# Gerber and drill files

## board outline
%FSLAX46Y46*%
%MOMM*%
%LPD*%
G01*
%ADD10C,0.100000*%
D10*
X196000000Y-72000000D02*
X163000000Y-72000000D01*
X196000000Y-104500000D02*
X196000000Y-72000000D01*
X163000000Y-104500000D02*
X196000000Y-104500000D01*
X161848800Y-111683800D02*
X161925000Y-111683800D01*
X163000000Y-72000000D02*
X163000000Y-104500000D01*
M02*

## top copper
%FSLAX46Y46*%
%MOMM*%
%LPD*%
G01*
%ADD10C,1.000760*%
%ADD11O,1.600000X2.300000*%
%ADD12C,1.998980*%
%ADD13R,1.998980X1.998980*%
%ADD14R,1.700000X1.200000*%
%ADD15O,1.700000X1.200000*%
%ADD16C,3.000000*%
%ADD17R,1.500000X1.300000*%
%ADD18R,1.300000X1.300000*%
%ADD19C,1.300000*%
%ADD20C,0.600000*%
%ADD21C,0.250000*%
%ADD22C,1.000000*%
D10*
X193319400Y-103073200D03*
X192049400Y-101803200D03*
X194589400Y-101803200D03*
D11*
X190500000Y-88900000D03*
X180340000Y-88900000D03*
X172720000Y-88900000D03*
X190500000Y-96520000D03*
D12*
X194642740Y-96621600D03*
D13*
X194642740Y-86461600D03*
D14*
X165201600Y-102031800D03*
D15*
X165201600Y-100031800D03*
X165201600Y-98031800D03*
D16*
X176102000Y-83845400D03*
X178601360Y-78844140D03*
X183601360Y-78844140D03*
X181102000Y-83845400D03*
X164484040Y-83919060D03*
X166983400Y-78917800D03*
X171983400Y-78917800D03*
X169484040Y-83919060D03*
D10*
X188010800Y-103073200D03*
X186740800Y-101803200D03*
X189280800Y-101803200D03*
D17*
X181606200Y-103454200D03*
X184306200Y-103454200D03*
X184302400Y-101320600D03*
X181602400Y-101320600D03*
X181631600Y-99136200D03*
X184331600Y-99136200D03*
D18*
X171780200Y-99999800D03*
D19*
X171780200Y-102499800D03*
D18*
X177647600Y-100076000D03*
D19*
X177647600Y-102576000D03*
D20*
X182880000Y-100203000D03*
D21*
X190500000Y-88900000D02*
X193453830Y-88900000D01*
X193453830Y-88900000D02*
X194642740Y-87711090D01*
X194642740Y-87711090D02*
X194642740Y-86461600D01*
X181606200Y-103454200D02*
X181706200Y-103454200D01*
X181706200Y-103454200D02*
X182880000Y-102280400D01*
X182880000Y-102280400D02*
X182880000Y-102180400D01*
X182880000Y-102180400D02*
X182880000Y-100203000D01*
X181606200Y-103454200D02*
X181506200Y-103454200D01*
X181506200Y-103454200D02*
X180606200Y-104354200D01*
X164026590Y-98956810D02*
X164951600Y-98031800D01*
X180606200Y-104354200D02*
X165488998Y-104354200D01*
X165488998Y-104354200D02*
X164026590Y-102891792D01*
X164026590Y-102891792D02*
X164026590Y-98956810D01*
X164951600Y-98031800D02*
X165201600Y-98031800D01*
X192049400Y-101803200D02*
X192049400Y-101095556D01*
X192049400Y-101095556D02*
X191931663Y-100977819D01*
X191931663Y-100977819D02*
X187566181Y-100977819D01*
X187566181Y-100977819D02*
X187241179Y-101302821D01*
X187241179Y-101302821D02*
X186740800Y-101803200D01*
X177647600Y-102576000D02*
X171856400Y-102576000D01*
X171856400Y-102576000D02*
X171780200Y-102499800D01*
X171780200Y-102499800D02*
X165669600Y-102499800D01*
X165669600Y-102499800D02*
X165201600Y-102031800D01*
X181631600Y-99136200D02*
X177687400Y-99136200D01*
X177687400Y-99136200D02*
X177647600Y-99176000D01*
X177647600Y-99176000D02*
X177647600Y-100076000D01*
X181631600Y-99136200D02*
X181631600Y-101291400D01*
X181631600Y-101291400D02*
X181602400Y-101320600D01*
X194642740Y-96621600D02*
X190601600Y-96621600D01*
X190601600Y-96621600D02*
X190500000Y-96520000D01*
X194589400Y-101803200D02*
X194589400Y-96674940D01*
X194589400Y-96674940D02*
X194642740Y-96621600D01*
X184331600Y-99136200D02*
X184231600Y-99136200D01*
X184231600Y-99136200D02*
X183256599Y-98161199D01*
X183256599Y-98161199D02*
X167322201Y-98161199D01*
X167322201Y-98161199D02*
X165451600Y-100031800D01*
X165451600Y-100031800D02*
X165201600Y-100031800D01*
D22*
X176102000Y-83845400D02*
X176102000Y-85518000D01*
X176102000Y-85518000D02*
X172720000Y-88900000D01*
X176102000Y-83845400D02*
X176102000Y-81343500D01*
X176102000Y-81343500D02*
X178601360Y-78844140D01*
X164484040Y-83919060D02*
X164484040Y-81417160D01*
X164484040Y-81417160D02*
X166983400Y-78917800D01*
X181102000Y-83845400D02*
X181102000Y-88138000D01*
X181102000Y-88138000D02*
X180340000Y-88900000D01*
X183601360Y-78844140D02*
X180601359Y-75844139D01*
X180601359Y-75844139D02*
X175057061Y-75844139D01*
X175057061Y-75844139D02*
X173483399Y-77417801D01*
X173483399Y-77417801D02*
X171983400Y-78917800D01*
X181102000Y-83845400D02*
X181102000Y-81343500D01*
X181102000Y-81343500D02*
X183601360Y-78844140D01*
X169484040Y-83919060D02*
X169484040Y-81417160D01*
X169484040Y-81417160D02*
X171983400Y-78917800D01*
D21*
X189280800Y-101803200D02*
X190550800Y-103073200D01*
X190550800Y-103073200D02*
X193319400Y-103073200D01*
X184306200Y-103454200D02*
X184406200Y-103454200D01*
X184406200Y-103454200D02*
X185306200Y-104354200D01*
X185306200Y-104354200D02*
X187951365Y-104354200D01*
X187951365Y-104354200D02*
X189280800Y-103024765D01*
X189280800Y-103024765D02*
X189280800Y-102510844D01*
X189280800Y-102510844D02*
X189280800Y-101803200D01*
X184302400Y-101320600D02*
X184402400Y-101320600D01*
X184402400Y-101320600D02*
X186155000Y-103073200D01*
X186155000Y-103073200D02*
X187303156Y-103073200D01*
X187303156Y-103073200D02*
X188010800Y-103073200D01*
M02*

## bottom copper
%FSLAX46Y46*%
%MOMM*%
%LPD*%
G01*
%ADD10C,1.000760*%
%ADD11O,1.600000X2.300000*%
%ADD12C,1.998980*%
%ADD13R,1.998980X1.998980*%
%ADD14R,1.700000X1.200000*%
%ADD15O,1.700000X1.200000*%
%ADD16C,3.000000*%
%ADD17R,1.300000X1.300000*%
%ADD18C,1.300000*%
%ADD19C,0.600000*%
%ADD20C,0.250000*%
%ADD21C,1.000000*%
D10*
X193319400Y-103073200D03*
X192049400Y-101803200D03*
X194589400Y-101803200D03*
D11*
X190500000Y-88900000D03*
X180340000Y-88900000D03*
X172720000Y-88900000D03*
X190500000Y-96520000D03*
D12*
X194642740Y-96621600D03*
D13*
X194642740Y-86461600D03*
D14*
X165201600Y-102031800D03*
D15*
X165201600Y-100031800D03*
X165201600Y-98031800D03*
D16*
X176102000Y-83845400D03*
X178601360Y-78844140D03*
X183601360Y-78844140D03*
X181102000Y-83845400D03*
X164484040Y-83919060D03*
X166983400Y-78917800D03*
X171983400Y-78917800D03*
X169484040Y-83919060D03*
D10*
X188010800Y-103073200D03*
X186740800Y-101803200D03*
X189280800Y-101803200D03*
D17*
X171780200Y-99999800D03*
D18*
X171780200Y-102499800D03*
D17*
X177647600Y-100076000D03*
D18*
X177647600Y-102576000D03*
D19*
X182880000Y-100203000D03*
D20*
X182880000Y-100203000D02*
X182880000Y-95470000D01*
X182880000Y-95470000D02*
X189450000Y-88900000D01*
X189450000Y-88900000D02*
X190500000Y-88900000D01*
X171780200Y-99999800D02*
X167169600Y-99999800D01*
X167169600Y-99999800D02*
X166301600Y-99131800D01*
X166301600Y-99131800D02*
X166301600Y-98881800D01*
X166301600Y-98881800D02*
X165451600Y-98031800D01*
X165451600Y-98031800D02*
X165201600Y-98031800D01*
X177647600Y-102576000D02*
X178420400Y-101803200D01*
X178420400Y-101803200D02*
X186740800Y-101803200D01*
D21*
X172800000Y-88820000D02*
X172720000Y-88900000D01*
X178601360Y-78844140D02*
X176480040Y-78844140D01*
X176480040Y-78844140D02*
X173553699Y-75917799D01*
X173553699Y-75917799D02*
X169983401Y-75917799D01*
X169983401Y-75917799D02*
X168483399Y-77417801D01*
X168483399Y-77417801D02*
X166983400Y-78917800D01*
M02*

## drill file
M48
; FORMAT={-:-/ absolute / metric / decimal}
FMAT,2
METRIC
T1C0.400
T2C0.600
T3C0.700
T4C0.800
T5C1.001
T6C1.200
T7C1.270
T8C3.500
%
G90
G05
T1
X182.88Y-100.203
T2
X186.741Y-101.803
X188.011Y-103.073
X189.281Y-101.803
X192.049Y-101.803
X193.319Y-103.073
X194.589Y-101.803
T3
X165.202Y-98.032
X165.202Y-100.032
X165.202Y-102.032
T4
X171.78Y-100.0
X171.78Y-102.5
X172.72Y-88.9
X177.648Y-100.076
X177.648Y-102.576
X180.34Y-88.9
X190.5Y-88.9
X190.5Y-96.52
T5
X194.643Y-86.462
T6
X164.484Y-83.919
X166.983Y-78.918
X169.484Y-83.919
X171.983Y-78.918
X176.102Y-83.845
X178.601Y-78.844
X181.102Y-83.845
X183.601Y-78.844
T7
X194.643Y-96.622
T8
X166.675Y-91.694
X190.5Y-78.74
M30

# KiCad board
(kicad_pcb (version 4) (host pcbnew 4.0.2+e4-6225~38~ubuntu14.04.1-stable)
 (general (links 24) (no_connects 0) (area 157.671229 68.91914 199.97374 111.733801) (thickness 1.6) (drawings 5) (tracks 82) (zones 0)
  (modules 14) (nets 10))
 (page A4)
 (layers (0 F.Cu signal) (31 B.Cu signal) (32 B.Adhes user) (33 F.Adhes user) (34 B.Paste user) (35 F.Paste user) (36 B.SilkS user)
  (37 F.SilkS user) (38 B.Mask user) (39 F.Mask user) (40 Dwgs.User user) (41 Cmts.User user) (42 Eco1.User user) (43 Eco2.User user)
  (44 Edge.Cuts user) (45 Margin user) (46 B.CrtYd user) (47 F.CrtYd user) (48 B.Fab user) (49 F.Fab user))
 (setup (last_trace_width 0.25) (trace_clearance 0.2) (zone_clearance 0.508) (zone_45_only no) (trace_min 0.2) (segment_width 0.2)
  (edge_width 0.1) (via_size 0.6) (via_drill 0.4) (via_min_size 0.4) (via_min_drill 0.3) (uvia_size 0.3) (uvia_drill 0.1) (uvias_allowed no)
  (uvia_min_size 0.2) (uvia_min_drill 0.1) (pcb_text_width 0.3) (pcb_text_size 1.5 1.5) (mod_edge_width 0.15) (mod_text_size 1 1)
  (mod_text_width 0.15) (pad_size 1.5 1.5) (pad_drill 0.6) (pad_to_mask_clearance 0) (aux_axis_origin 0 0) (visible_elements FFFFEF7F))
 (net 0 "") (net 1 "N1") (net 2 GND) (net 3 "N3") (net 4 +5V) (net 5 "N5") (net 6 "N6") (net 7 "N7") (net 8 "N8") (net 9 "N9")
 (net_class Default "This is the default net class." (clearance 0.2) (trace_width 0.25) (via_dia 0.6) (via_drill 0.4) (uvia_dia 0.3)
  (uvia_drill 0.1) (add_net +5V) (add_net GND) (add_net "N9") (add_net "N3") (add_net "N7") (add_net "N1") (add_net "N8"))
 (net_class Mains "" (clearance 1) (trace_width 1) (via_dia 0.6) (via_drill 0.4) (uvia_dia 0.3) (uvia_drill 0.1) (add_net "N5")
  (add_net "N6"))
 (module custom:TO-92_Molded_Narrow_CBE (layer F.Cu) (at 194.5894 101.8032 180)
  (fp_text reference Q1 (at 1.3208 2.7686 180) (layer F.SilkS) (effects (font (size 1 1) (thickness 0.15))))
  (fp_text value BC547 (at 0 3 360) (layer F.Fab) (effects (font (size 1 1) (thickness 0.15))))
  (pad 2 thru_hole circle (at 1.27 -1.27 270) (size 1.00076 1.00076) (drill 0.6) (layers *.Cu *.Mask F.SilkS) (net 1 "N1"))
  (pad 3 thru_hole circle (at 2.54 0 270) (size 1.00076 1.00076) (drill 0.6) (layers *.Cu *.Mask F.SilkS) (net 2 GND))
  (pad 1 thru_hole circle (at 0 0 270) (size 1.00076 1.00076) (drill 0.6) (layers *.Cu *.Mask F.SilkS) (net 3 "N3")))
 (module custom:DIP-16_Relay (layer F.Cu) (at 190.5 88.9 270)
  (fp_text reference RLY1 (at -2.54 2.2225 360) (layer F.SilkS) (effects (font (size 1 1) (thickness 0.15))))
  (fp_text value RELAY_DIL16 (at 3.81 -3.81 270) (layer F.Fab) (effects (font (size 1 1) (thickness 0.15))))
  (pad 1 thru_hole oval (at 0 0 270) (size 2.3 1.6) (drill 0.8) (layers *.Cu *.Mask F.SilkS) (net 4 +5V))
  (pad 5 thru_hole oval (at 0 10.16 270) (size 2.3 1.6) (drill 0.8) (layers *.Cu *.Mask F.SilkS) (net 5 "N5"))
  (pad 8 thru_hole oval (at 0 17.78 270) (size 2.3 1.6) (drill 0.8) (layers *.Cu *.Mask F.SilkS) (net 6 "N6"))
  (pad 16 thru_hole oval (at 7.62 0 270) (size 2.3 1.6) (drill 0.8) (layers *.Cu *.Mask F.SilkS) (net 3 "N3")))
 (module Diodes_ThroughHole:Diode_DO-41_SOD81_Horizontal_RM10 (layer F.Cu) (at 194.6402 86.4616 270)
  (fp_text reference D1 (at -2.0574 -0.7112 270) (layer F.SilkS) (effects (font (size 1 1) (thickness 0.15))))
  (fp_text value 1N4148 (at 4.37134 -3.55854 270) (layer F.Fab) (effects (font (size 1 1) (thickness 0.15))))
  (pad 2 thru_hole circle (at 10.16 -0.00254 90) (size 1.99898 1.99898) (drill 1.27) (layers *.Cu *.Mask F.SilkS) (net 3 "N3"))
  (pad 1 thru_hole rect (at 0 -0.00254 90) (size 1.99898 1.99898) (drill 1.00076) (layers *.Cu *.Mask F.SilkS) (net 4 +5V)))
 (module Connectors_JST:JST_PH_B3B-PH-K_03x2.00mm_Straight (layer F.Cu) (at 165.2016 102.0318 90)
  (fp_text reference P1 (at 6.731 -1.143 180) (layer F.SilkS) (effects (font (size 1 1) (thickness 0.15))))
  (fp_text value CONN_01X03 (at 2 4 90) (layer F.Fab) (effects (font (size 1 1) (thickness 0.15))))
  (pad 1 thru_hole rect (at 0 0 90) (size 1.2 1.7) (drill 0.7) (layers *.Cu *.Mask F.SilkS) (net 2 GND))
  (pad 2 thru_hole oval (at 2 0 90) (size 1.2 1.7) (drill 0.7) (layers *.Cu *.Mask F.SilkS) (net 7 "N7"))
  (pad 3 thru_hole oval (at 4 0 90) (size 1.2 1.7) (drill 0.7) (layers *.Cu *.Mask F.SilkS) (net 4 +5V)))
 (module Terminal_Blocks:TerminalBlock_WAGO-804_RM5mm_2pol (layer F.Cu) (at 183.60136 78.84414 180)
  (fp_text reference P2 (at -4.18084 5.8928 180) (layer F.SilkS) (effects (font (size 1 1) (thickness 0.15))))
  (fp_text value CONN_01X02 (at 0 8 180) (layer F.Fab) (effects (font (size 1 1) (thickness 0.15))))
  (pad 2 thru_hole circle (at 7.49936 -5.00126 180) (size 3 3) (drill 1.2) (layers *.Cu *.Mask F.SilkS) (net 6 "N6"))
  (pad 2 thru_hole circle (at 5 0 180) (size 3 3) (drill 1.2) (layers *.Cu *.Mask F.SilkS) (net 6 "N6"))
  (pad 1 thru_hole circle (at 0 0 180) (size 3 3) (drill 1.2) (layers *.Cu *.Mask F.SilkS) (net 5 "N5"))
  (pad 1 thru_hole circle (at 2.49936 -5.00126 180) (size 3 3) (drill 1.2) (layers *.Cu *.Mask F.SilkS) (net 5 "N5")))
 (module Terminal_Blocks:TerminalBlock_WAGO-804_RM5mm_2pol (layer F.Cu) (at 171.9834 78.9178 180)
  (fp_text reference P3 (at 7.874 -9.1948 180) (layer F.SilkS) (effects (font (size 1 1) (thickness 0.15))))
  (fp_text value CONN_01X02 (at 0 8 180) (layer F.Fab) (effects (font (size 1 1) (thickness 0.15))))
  (pad 2 thru_hole circle (at 7.49936 -5.00126 180) (size 3 3) (drill 1.2) (layers *.Cu *.Mask F.SilkS) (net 6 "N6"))
  (pad 2 thru_hole circle (at 5 0 180) (size 3 3) (drill 1.2) (layers *.Cu *.Mask F.SilkS) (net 6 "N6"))
  (pad 1 thru_hole circle (at 0 0 180) (size 3 3) (drill 1.2) (layers *.Cu *.Mask F.SilkS) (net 5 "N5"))
  (pad 1 thru_hole circle (at 2.49936 -5.00126 180) (size 3 3) (drill 1.2) (layers *.Cu *.Mask F.SilkS) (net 5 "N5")))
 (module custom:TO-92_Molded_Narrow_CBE (layer F.Cu) (at 189.2808 101.8032 180)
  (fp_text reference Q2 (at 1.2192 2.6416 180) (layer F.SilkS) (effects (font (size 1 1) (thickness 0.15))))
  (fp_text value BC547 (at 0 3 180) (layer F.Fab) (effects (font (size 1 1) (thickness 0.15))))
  (pad 2 thru_hole circle (at 1.27 -1.27 270) (size 1.00076 1.00076) (drill 0.6) (layers *.Cu *.Mask F.SilkS) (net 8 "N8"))
  (pad 3 thru_hole circle (at 2.54 0 270) (size 1.00076 1.00076) (drill 0.6) (layers *.Cu *.Mask F.SilkS) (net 2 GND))
  (pad 1 thru_hole circle (at 0 0 270) (size 1.00076 1.00076) (drill 0.6) (layers *.Cu *.Mask F.SilkS) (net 1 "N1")))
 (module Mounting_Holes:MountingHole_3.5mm (layer F.Cu) (at 190.5 78.74)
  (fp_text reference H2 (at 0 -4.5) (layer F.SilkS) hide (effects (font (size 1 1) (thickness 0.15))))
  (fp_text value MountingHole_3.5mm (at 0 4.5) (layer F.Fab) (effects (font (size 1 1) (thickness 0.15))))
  (pad 1 np_thru_hole circle (at 0 0) (size 3.5 3.5) (drill 3.5) (layers *.Cu *.Mask F.SilkS)))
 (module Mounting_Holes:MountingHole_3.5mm (layer F.Cu) (at 166.6748 91.694)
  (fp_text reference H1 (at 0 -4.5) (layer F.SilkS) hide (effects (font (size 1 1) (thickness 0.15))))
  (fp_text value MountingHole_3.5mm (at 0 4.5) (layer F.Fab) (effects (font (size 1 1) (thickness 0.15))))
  (pad 1 np_thru_hole circle (at 0 0) (size 3.5 3.5) (drill 3.5) (layers *.Cu *.Mask F.SilkS)))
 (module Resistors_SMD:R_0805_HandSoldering (layer F.Cu) (at 182.9562 103.4542)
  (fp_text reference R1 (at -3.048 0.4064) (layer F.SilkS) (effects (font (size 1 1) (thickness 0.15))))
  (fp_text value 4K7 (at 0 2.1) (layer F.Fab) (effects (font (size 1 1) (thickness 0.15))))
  (pad 1 smd rect (at -1.35 0) (size 1.5 1.3) (layers F.Cu F.Paste F.Mask) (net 4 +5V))
  (pad 2 smd rect (at 1.35 0) (size 1.5 1.3) (layers F.Cu F.Paste F.Mask) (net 1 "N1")))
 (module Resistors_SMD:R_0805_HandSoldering (layer F.Cu) (at 182.9524 101.3206 180)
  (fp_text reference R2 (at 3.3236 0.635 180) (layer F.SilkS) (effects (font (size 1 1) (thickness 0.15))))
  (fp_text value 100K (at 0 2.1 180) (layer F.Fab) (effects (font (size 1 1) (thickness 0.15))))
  (pad 1 smd rect (at -1.35 0 180) (size 1.5 1.3) (layers F.Cu F.Paste F.Mask) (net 8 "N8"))
  (pad 2 smd rect (at 1.35 0 180) (size 1.5 1.3) (layers F.Cu F.Paste F.Mask) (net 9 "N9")))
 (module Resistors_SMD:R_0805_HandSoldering (layer F.Cu) (at 182.9816 99.1362)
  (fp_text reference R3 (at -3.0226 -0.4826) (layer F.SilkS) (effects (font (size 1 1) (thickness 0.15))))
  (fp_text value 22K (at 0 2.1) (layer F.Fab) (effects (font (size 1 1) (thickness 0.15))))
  (pad 1 smd rect (at -1.35 0) (size 1.5 1.3) (layers F.Cu F.Paste F.Mask) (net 9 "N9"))
  (pad 2 smd rect (at 1.35 0) (size 1.5 1.3) (layers F.Cu F.Paste F.Mask) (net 7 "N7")))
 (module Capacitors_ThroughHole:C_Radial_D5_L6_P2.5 (layer F.Cu) (at 171.7802 99.9998 270)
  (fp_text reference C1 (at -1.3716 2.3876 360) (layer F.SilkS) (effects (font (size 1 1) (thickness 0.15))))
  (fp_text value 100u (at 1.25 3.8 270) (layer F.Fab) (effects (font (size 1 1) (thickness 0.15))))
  (pad 1 thru_hole rect (at 0 0 270) (size 1.3 1.3) (drill 0.8) (layers *.Cu *.Mask F.SilkS) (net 4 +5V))
  (pad 2 thru_hole circle (at 2.5 0 270) (size 1.3 1.3) (drill 0.8) (layers *.Cu *.Mask F.SilkS) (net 2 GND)))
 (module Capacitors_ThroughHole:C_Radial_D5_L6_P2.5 (layer F.Cu) (at 177.6476 100.076 270)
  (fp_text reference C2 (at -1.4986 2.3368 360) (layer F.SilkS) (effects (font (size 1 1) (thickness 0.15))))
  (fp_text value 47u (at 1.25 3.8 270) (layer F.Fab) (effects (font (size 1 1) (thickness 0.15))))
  (pad 1 thru_hole rect (at 0 0 270) (size 1.3 1.3) (drill 0.8) (layers *.Cu *.Mask F.SilkS) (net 9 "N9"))
  (pad 2 thru_hole circle (at 2.5 0 270) (size 1.3 1.3) (drill 0.8) (layers *.Cu *.Mask F.SilkS) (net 2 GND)))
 (gr_line (start 196 72) (end 163 72) (angle 90) (layer Edge.Cuts) (width 0.1))
 (gr_line (start 196 104.5) (end 196 72) (angle 90) (layer Edge.Cuts) (width 0.1))
 (gr_line (start 163 104.5) (end 196 104.5) (angle 90) (layer Edge.Cuts) (width 0.1))
 (gr_line (start 161.8488 111.6838) (end 161.925 111.6838) (angle 90) (layer Edge.Cuts) (width 0.1))
 (gr_line (start 163 72) (end 163 104.5) (angle 90) (layer Edge.Cuts) (width 0.1))
 (segment (start 190.5 88.9) (end 193.45383 88.9) (width 0.25) (layer F.Cu) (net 4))
 (segment (start 193.45383 88.9) (end 194.64274 87.71109) (width 0.25) (layer F.Cu) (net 4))
 (segment (start 194.64274 87.71109) (end 194.64274 86.4616) (width 0.25) (layer F.Cu) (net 4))
 (segment (start 182.88 100.203) (end 182.88 95.47) (width 0.25) (layer B.Cu) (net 4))
 (segment (start 182.88 95.47) (end 189.45 88.9) (width 0.25) (layer B.Cu) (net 4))
 (segment (start 189.45 88.9) (end 190.5 88.9) (width 0.25) (layer B.Cu) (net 4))
 (segment (start 181.6062 103.4542) (end 181.7062 103.4542) (width 0.25) (layer F.Cu) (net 4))
 (segment (start 181.7062 103.4542) (end 182.88 102.2804) (width 0.25) (layer F.Cu) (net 4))
 (segment (start 182.88 102.2804) (end 182.88 102.1804) (width 0.25) (layer F.Cu) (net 4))
 (segment (start 182.88 102.1804) (end 182.88 100.203) (width 0.25) (layer F.Cu) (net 4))
 (via (at 182.88 100.203) (size 0.6) (drill 0.4) (layers F.Cu B.Cu) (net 4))
 (segment (start 171.7802 99.9998) (end 167.1696 99.9998) (width 0.25) (layer B.Cu) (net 4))
 (segment (start 167.1696 99.9998) (end 166.3016 99.1318) (width 0.25) (layer B.Cu) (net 4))
 (segment (start 166.3016 99.1318) (end 166.3016 98.8818) (width 0.25) (layer B.Cu) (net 4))
 (segment (start 166.3016 98.8818) (end 165.4516 98.0318) (width 0.25) (layer B.Cu) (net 4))
 (segment (start 165.4516 98.0318) (end 165.2016 98.0318) (width 0.25) (layer B.Cu) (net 4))
 (segment (start 181.6062 103.4542) (end 181.5062 103.4542) (width 0.25) (layer F.Cu) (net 4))
 (segment (start 181.5062 103.4542) (end 180.6062 104.3542) (width 0.25) (layer F.Cu) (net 4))
 (segment (start 164.02659 98.95681) (end 164.9516 98.0318) (width 0.25) (layer F.Cu) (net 4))
 (segment (start 180.6062 104.3542) (end 165.488998 104.3542) (width 0.25) (layer F.Cu) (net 4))
 (segment (start 165.488998 104.3542) (end 164.02659 102.891792) (width 0.25) (layer F.Cu) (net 4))
 (segment (start 164.02659 102.891792) (end 164.02659 98.95681) (width 0.25) (layer F.Cu) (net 4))
 (segment (start 164.9516 98.0318) (end 165.2016 98.0318) (width 0.25) (layer F.Cu) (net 4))
 (segment (start 192.0494 101.8032) (end 192.0494 101.095556) (width 0.25) (layer F.Cu) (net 2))
 (segment (start 192.0494 101.095556) (end 191.931663 100.977819) (width 0.25) (layer F.Cu) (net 2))
 (segment (start 191.931663 100.977819) (end 187.566181 100.977819) (width 0.25) (layer F.Cu) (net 2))
 (segment (start 187.566181 100.977819) (end 187.241179 101.302821) (width 0.25) (layer F.Cu) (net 2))
 (segment (start 187.241179 101.302821) (end 186.7408 101.8032) (width 0.25) (layer F.Cu) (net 2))
 (segment (start 177.6476 102.576) (end 178.4204 101.8032) (width 0.25) (layer B.Cu) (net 2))
 (segment (start 178.4204 101.8032) (end 186.7408 101.8032) (width 0.25) (layer B.Cu) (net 2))
 (segment (start 177.6476 102.576) (end 171.8564 102.576) (width 0.25) (layer F.Cu) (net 2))
 (segment (start 171.8564 102.576) (end 171.7802 102.4998) (width 0.25) (layer F.Cu) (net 2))
 (segment (start 171.7802 102.4998) (end 165.6696 102.4998) (width 0.25) (layer F.Cu) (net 2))
 (segment (start 165.6696 102.4998) (end 165.2016 102.0318) (width 0.25) (layer F.Cu) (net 2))
 (segment (start 181.6316 99.1362) (end 177.6874 99.1362) (width 0.25) (layer F.Cu) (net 9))
 (segment (start 177.6874 99.1362) (end 177.6476 99.176) (width 0.25) (layer F.Cu) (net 9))
 (segment (start 177.6476 99.176) (end 177.6476 100.076) (width 0.25) (layer F.Cu) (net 9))
 (segment (start 181.6316 99.1362) (end 181.6316 101.2914) (width 0.25) (layer F.Cu) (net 9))
 (segment (start 181.6316 101.2914) (end 181.6024 101.3206) (width 0.25) (layer F.Cu) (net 9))
 (segment (start 194.64274 96.6216) (end 190.6016 96.6216) (width 0.25) (layer F.Cu) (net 3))
 (segment (start 190.6016 96.6216) (end 190.5 96.52) (width 0.25) (layer F.Cu) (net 3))
 (segment (start 194.5894 101.8032) (end 194.5894 96.67494) (width 0.25) (layer F.Cu) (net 3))
 (segment (start 194.5894 96.67494) (end 194.64274 96.6216) (width 0.25) (layer F.Cu) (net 3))
 (segment (start 184.3316 99.1362) (end 184.2316 99.1362) (width 0.25) (layer F.Cu) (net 7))
 (segment (start 184.2316 99.1362) (end 183.256599 98.161199) (width 0.25) (layer F.Cu) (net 7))
 (segment (start 183.256599 98.161199) (end 167.322201 98.161199) (width 0.25) (layer F.Cu) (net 7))
 (segment (start 167.322201 98.161199) (end 165.4516 100.0318) (width 0.25) (layer F.Cu) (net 7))
 (segment (start 165.4516 100.0318) (end 165.2016 100.0318) (width 0.25) (layer F.Cu) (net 7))
 (segment (start 172.8 88.82) (end 172.72 88.9) (width 1) (layer B.Cu) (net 6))
 (segment (start 176.102 83.8454) (end 176.102 85.518) (width 1) (layer F.Cu) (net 6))
 (segment (start 176.102 85.518) (end 172.72 88.9) (width 1) (layer F.Cu) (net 6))
 (segment (start 178.60136 78.84414) (end 176.48004 78.84414) (width 1) (layer B.Cu) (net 6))
 (segment (start 176.48004 78.84414) (end 173.553699 75.917799) (width 1) (layer B.Cu) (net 6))
 (segment (start 173.553699 75.917799) (end 169.983401 75.917799) (width 1) (layer B.Cu) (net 6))
 (segment (start 169.983401 75.917799) (end 168.483399 77.417801) (width 1) (layer B.Cu) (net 6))
 (segment (start 168.483399 77.417801) (end 166.9834 78.9178) (width 1) (layer B.Cu) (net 6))
 (segment (start 176.102 83.8454) (end 176.102 81.3435) (width 1) (layer F.Cu) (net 6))
 (segment (start 176.102 81.3435) (end 178.60136 78.84414) (width 1) (layer F.Cu) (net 6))
 (segment (start 164.48404 83.91906) (end 164.48404 81.41716) (width 1) (layer F.Cu) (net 6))
 (segment (start 164.48404 81.41716) (end 166.9834 78.9178) (width 1) (layer F.Cu) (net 6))
 (segment (start 181.102 83.8454) (end 181.102 88.138) (width 1) (layer F.Cu) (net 5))
 (segment (start 181.102 88.138) (end 180.34 88.9) (width 1) (layer F.Cu) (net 5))
 (segment (start 183.60136 78.84414) (end 180.601359 75.844139) (width 1) (layer F.Cu) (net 5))
 (segment (start 180.601359 75.844139) (end 175.057061 75.844139) (width 1) (layer F.Cu) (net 5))
 (segment (start 175.057061 75.844139) (end 173.483399 77.417801) (width 1) (layer F.Cu) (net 5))
 (segment (start 173.483399 77.417801) (end 171.9834 78.9178) (width 1) (layer F.Cu) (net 5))
 (segment (start 181.102 83.8454) (end 181.102 81.3435) (width 1) (layer F.Cu) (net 5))
 (segment (start 181.102 81.3435) (end 183.60136 78.84414) (width 1) (layer F.Cu) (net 5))
 (segment (start 169.48404 83.91906) (end 169.48404 81.41716) (width 1) (layer F.Cu) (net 5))
 (segment (start 169.48404 81.41716) (end 171.9834 78.9178) (width 1) (layer F.Cu) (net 5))
 (segment (start 189.2808 101.8032) (end 190.5508 103.0732) (width 0.25) (layer F.Cu) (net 1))
 (segment (start 190.5508 103.0732) (end 193.3194 103.0732) (width 0.25) (layer F.Cu) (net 1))
 (segment (start 184.3062 103.4542) (end 184.4062 103.4542) (width 0.25) (layer F.Cu) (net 1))
 (segment (start 184.4062 103.4542) (end 185.3062 104.3542) (width 0.25) (layer F.Cu) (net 1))
 (segment (start 185.3062 104.3542) (end 187.951365 104.3542) (width 0.25) (layer F.Cu) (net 1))
 (segment (start 187.951365 104.3542) (end 189.2808 103.024765) (width 0.25) (layer F.Cu) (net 1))
 (segment (start 189.2808 103.024765) (end 189.2808 102.510844) (width 0.25) (layer F.Cu) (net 1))
 (segment (start 189.2808 102.510844) (end 189.2808 101.8032) (width 0.25) (layer F.Cu) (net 1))
 (segment (start 184.3024 101.3206) (end 184.4024 101.3206) (width 0.25) (layer F.Cu) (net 8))
 (segment (start 184.4024 101.3206) (end 186.155 103.0732) (width 0.25) (layer F.Cu) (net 8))
 (segment (start 186.155 103.0732) (end 187.303156 103.0732) (width 0.25) (layer F.Cu) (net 8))
 (segment (start 187.303156 103.0732) (end 188.0108 103.0732) (width 0.25) (layer F.Cu) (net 8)))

